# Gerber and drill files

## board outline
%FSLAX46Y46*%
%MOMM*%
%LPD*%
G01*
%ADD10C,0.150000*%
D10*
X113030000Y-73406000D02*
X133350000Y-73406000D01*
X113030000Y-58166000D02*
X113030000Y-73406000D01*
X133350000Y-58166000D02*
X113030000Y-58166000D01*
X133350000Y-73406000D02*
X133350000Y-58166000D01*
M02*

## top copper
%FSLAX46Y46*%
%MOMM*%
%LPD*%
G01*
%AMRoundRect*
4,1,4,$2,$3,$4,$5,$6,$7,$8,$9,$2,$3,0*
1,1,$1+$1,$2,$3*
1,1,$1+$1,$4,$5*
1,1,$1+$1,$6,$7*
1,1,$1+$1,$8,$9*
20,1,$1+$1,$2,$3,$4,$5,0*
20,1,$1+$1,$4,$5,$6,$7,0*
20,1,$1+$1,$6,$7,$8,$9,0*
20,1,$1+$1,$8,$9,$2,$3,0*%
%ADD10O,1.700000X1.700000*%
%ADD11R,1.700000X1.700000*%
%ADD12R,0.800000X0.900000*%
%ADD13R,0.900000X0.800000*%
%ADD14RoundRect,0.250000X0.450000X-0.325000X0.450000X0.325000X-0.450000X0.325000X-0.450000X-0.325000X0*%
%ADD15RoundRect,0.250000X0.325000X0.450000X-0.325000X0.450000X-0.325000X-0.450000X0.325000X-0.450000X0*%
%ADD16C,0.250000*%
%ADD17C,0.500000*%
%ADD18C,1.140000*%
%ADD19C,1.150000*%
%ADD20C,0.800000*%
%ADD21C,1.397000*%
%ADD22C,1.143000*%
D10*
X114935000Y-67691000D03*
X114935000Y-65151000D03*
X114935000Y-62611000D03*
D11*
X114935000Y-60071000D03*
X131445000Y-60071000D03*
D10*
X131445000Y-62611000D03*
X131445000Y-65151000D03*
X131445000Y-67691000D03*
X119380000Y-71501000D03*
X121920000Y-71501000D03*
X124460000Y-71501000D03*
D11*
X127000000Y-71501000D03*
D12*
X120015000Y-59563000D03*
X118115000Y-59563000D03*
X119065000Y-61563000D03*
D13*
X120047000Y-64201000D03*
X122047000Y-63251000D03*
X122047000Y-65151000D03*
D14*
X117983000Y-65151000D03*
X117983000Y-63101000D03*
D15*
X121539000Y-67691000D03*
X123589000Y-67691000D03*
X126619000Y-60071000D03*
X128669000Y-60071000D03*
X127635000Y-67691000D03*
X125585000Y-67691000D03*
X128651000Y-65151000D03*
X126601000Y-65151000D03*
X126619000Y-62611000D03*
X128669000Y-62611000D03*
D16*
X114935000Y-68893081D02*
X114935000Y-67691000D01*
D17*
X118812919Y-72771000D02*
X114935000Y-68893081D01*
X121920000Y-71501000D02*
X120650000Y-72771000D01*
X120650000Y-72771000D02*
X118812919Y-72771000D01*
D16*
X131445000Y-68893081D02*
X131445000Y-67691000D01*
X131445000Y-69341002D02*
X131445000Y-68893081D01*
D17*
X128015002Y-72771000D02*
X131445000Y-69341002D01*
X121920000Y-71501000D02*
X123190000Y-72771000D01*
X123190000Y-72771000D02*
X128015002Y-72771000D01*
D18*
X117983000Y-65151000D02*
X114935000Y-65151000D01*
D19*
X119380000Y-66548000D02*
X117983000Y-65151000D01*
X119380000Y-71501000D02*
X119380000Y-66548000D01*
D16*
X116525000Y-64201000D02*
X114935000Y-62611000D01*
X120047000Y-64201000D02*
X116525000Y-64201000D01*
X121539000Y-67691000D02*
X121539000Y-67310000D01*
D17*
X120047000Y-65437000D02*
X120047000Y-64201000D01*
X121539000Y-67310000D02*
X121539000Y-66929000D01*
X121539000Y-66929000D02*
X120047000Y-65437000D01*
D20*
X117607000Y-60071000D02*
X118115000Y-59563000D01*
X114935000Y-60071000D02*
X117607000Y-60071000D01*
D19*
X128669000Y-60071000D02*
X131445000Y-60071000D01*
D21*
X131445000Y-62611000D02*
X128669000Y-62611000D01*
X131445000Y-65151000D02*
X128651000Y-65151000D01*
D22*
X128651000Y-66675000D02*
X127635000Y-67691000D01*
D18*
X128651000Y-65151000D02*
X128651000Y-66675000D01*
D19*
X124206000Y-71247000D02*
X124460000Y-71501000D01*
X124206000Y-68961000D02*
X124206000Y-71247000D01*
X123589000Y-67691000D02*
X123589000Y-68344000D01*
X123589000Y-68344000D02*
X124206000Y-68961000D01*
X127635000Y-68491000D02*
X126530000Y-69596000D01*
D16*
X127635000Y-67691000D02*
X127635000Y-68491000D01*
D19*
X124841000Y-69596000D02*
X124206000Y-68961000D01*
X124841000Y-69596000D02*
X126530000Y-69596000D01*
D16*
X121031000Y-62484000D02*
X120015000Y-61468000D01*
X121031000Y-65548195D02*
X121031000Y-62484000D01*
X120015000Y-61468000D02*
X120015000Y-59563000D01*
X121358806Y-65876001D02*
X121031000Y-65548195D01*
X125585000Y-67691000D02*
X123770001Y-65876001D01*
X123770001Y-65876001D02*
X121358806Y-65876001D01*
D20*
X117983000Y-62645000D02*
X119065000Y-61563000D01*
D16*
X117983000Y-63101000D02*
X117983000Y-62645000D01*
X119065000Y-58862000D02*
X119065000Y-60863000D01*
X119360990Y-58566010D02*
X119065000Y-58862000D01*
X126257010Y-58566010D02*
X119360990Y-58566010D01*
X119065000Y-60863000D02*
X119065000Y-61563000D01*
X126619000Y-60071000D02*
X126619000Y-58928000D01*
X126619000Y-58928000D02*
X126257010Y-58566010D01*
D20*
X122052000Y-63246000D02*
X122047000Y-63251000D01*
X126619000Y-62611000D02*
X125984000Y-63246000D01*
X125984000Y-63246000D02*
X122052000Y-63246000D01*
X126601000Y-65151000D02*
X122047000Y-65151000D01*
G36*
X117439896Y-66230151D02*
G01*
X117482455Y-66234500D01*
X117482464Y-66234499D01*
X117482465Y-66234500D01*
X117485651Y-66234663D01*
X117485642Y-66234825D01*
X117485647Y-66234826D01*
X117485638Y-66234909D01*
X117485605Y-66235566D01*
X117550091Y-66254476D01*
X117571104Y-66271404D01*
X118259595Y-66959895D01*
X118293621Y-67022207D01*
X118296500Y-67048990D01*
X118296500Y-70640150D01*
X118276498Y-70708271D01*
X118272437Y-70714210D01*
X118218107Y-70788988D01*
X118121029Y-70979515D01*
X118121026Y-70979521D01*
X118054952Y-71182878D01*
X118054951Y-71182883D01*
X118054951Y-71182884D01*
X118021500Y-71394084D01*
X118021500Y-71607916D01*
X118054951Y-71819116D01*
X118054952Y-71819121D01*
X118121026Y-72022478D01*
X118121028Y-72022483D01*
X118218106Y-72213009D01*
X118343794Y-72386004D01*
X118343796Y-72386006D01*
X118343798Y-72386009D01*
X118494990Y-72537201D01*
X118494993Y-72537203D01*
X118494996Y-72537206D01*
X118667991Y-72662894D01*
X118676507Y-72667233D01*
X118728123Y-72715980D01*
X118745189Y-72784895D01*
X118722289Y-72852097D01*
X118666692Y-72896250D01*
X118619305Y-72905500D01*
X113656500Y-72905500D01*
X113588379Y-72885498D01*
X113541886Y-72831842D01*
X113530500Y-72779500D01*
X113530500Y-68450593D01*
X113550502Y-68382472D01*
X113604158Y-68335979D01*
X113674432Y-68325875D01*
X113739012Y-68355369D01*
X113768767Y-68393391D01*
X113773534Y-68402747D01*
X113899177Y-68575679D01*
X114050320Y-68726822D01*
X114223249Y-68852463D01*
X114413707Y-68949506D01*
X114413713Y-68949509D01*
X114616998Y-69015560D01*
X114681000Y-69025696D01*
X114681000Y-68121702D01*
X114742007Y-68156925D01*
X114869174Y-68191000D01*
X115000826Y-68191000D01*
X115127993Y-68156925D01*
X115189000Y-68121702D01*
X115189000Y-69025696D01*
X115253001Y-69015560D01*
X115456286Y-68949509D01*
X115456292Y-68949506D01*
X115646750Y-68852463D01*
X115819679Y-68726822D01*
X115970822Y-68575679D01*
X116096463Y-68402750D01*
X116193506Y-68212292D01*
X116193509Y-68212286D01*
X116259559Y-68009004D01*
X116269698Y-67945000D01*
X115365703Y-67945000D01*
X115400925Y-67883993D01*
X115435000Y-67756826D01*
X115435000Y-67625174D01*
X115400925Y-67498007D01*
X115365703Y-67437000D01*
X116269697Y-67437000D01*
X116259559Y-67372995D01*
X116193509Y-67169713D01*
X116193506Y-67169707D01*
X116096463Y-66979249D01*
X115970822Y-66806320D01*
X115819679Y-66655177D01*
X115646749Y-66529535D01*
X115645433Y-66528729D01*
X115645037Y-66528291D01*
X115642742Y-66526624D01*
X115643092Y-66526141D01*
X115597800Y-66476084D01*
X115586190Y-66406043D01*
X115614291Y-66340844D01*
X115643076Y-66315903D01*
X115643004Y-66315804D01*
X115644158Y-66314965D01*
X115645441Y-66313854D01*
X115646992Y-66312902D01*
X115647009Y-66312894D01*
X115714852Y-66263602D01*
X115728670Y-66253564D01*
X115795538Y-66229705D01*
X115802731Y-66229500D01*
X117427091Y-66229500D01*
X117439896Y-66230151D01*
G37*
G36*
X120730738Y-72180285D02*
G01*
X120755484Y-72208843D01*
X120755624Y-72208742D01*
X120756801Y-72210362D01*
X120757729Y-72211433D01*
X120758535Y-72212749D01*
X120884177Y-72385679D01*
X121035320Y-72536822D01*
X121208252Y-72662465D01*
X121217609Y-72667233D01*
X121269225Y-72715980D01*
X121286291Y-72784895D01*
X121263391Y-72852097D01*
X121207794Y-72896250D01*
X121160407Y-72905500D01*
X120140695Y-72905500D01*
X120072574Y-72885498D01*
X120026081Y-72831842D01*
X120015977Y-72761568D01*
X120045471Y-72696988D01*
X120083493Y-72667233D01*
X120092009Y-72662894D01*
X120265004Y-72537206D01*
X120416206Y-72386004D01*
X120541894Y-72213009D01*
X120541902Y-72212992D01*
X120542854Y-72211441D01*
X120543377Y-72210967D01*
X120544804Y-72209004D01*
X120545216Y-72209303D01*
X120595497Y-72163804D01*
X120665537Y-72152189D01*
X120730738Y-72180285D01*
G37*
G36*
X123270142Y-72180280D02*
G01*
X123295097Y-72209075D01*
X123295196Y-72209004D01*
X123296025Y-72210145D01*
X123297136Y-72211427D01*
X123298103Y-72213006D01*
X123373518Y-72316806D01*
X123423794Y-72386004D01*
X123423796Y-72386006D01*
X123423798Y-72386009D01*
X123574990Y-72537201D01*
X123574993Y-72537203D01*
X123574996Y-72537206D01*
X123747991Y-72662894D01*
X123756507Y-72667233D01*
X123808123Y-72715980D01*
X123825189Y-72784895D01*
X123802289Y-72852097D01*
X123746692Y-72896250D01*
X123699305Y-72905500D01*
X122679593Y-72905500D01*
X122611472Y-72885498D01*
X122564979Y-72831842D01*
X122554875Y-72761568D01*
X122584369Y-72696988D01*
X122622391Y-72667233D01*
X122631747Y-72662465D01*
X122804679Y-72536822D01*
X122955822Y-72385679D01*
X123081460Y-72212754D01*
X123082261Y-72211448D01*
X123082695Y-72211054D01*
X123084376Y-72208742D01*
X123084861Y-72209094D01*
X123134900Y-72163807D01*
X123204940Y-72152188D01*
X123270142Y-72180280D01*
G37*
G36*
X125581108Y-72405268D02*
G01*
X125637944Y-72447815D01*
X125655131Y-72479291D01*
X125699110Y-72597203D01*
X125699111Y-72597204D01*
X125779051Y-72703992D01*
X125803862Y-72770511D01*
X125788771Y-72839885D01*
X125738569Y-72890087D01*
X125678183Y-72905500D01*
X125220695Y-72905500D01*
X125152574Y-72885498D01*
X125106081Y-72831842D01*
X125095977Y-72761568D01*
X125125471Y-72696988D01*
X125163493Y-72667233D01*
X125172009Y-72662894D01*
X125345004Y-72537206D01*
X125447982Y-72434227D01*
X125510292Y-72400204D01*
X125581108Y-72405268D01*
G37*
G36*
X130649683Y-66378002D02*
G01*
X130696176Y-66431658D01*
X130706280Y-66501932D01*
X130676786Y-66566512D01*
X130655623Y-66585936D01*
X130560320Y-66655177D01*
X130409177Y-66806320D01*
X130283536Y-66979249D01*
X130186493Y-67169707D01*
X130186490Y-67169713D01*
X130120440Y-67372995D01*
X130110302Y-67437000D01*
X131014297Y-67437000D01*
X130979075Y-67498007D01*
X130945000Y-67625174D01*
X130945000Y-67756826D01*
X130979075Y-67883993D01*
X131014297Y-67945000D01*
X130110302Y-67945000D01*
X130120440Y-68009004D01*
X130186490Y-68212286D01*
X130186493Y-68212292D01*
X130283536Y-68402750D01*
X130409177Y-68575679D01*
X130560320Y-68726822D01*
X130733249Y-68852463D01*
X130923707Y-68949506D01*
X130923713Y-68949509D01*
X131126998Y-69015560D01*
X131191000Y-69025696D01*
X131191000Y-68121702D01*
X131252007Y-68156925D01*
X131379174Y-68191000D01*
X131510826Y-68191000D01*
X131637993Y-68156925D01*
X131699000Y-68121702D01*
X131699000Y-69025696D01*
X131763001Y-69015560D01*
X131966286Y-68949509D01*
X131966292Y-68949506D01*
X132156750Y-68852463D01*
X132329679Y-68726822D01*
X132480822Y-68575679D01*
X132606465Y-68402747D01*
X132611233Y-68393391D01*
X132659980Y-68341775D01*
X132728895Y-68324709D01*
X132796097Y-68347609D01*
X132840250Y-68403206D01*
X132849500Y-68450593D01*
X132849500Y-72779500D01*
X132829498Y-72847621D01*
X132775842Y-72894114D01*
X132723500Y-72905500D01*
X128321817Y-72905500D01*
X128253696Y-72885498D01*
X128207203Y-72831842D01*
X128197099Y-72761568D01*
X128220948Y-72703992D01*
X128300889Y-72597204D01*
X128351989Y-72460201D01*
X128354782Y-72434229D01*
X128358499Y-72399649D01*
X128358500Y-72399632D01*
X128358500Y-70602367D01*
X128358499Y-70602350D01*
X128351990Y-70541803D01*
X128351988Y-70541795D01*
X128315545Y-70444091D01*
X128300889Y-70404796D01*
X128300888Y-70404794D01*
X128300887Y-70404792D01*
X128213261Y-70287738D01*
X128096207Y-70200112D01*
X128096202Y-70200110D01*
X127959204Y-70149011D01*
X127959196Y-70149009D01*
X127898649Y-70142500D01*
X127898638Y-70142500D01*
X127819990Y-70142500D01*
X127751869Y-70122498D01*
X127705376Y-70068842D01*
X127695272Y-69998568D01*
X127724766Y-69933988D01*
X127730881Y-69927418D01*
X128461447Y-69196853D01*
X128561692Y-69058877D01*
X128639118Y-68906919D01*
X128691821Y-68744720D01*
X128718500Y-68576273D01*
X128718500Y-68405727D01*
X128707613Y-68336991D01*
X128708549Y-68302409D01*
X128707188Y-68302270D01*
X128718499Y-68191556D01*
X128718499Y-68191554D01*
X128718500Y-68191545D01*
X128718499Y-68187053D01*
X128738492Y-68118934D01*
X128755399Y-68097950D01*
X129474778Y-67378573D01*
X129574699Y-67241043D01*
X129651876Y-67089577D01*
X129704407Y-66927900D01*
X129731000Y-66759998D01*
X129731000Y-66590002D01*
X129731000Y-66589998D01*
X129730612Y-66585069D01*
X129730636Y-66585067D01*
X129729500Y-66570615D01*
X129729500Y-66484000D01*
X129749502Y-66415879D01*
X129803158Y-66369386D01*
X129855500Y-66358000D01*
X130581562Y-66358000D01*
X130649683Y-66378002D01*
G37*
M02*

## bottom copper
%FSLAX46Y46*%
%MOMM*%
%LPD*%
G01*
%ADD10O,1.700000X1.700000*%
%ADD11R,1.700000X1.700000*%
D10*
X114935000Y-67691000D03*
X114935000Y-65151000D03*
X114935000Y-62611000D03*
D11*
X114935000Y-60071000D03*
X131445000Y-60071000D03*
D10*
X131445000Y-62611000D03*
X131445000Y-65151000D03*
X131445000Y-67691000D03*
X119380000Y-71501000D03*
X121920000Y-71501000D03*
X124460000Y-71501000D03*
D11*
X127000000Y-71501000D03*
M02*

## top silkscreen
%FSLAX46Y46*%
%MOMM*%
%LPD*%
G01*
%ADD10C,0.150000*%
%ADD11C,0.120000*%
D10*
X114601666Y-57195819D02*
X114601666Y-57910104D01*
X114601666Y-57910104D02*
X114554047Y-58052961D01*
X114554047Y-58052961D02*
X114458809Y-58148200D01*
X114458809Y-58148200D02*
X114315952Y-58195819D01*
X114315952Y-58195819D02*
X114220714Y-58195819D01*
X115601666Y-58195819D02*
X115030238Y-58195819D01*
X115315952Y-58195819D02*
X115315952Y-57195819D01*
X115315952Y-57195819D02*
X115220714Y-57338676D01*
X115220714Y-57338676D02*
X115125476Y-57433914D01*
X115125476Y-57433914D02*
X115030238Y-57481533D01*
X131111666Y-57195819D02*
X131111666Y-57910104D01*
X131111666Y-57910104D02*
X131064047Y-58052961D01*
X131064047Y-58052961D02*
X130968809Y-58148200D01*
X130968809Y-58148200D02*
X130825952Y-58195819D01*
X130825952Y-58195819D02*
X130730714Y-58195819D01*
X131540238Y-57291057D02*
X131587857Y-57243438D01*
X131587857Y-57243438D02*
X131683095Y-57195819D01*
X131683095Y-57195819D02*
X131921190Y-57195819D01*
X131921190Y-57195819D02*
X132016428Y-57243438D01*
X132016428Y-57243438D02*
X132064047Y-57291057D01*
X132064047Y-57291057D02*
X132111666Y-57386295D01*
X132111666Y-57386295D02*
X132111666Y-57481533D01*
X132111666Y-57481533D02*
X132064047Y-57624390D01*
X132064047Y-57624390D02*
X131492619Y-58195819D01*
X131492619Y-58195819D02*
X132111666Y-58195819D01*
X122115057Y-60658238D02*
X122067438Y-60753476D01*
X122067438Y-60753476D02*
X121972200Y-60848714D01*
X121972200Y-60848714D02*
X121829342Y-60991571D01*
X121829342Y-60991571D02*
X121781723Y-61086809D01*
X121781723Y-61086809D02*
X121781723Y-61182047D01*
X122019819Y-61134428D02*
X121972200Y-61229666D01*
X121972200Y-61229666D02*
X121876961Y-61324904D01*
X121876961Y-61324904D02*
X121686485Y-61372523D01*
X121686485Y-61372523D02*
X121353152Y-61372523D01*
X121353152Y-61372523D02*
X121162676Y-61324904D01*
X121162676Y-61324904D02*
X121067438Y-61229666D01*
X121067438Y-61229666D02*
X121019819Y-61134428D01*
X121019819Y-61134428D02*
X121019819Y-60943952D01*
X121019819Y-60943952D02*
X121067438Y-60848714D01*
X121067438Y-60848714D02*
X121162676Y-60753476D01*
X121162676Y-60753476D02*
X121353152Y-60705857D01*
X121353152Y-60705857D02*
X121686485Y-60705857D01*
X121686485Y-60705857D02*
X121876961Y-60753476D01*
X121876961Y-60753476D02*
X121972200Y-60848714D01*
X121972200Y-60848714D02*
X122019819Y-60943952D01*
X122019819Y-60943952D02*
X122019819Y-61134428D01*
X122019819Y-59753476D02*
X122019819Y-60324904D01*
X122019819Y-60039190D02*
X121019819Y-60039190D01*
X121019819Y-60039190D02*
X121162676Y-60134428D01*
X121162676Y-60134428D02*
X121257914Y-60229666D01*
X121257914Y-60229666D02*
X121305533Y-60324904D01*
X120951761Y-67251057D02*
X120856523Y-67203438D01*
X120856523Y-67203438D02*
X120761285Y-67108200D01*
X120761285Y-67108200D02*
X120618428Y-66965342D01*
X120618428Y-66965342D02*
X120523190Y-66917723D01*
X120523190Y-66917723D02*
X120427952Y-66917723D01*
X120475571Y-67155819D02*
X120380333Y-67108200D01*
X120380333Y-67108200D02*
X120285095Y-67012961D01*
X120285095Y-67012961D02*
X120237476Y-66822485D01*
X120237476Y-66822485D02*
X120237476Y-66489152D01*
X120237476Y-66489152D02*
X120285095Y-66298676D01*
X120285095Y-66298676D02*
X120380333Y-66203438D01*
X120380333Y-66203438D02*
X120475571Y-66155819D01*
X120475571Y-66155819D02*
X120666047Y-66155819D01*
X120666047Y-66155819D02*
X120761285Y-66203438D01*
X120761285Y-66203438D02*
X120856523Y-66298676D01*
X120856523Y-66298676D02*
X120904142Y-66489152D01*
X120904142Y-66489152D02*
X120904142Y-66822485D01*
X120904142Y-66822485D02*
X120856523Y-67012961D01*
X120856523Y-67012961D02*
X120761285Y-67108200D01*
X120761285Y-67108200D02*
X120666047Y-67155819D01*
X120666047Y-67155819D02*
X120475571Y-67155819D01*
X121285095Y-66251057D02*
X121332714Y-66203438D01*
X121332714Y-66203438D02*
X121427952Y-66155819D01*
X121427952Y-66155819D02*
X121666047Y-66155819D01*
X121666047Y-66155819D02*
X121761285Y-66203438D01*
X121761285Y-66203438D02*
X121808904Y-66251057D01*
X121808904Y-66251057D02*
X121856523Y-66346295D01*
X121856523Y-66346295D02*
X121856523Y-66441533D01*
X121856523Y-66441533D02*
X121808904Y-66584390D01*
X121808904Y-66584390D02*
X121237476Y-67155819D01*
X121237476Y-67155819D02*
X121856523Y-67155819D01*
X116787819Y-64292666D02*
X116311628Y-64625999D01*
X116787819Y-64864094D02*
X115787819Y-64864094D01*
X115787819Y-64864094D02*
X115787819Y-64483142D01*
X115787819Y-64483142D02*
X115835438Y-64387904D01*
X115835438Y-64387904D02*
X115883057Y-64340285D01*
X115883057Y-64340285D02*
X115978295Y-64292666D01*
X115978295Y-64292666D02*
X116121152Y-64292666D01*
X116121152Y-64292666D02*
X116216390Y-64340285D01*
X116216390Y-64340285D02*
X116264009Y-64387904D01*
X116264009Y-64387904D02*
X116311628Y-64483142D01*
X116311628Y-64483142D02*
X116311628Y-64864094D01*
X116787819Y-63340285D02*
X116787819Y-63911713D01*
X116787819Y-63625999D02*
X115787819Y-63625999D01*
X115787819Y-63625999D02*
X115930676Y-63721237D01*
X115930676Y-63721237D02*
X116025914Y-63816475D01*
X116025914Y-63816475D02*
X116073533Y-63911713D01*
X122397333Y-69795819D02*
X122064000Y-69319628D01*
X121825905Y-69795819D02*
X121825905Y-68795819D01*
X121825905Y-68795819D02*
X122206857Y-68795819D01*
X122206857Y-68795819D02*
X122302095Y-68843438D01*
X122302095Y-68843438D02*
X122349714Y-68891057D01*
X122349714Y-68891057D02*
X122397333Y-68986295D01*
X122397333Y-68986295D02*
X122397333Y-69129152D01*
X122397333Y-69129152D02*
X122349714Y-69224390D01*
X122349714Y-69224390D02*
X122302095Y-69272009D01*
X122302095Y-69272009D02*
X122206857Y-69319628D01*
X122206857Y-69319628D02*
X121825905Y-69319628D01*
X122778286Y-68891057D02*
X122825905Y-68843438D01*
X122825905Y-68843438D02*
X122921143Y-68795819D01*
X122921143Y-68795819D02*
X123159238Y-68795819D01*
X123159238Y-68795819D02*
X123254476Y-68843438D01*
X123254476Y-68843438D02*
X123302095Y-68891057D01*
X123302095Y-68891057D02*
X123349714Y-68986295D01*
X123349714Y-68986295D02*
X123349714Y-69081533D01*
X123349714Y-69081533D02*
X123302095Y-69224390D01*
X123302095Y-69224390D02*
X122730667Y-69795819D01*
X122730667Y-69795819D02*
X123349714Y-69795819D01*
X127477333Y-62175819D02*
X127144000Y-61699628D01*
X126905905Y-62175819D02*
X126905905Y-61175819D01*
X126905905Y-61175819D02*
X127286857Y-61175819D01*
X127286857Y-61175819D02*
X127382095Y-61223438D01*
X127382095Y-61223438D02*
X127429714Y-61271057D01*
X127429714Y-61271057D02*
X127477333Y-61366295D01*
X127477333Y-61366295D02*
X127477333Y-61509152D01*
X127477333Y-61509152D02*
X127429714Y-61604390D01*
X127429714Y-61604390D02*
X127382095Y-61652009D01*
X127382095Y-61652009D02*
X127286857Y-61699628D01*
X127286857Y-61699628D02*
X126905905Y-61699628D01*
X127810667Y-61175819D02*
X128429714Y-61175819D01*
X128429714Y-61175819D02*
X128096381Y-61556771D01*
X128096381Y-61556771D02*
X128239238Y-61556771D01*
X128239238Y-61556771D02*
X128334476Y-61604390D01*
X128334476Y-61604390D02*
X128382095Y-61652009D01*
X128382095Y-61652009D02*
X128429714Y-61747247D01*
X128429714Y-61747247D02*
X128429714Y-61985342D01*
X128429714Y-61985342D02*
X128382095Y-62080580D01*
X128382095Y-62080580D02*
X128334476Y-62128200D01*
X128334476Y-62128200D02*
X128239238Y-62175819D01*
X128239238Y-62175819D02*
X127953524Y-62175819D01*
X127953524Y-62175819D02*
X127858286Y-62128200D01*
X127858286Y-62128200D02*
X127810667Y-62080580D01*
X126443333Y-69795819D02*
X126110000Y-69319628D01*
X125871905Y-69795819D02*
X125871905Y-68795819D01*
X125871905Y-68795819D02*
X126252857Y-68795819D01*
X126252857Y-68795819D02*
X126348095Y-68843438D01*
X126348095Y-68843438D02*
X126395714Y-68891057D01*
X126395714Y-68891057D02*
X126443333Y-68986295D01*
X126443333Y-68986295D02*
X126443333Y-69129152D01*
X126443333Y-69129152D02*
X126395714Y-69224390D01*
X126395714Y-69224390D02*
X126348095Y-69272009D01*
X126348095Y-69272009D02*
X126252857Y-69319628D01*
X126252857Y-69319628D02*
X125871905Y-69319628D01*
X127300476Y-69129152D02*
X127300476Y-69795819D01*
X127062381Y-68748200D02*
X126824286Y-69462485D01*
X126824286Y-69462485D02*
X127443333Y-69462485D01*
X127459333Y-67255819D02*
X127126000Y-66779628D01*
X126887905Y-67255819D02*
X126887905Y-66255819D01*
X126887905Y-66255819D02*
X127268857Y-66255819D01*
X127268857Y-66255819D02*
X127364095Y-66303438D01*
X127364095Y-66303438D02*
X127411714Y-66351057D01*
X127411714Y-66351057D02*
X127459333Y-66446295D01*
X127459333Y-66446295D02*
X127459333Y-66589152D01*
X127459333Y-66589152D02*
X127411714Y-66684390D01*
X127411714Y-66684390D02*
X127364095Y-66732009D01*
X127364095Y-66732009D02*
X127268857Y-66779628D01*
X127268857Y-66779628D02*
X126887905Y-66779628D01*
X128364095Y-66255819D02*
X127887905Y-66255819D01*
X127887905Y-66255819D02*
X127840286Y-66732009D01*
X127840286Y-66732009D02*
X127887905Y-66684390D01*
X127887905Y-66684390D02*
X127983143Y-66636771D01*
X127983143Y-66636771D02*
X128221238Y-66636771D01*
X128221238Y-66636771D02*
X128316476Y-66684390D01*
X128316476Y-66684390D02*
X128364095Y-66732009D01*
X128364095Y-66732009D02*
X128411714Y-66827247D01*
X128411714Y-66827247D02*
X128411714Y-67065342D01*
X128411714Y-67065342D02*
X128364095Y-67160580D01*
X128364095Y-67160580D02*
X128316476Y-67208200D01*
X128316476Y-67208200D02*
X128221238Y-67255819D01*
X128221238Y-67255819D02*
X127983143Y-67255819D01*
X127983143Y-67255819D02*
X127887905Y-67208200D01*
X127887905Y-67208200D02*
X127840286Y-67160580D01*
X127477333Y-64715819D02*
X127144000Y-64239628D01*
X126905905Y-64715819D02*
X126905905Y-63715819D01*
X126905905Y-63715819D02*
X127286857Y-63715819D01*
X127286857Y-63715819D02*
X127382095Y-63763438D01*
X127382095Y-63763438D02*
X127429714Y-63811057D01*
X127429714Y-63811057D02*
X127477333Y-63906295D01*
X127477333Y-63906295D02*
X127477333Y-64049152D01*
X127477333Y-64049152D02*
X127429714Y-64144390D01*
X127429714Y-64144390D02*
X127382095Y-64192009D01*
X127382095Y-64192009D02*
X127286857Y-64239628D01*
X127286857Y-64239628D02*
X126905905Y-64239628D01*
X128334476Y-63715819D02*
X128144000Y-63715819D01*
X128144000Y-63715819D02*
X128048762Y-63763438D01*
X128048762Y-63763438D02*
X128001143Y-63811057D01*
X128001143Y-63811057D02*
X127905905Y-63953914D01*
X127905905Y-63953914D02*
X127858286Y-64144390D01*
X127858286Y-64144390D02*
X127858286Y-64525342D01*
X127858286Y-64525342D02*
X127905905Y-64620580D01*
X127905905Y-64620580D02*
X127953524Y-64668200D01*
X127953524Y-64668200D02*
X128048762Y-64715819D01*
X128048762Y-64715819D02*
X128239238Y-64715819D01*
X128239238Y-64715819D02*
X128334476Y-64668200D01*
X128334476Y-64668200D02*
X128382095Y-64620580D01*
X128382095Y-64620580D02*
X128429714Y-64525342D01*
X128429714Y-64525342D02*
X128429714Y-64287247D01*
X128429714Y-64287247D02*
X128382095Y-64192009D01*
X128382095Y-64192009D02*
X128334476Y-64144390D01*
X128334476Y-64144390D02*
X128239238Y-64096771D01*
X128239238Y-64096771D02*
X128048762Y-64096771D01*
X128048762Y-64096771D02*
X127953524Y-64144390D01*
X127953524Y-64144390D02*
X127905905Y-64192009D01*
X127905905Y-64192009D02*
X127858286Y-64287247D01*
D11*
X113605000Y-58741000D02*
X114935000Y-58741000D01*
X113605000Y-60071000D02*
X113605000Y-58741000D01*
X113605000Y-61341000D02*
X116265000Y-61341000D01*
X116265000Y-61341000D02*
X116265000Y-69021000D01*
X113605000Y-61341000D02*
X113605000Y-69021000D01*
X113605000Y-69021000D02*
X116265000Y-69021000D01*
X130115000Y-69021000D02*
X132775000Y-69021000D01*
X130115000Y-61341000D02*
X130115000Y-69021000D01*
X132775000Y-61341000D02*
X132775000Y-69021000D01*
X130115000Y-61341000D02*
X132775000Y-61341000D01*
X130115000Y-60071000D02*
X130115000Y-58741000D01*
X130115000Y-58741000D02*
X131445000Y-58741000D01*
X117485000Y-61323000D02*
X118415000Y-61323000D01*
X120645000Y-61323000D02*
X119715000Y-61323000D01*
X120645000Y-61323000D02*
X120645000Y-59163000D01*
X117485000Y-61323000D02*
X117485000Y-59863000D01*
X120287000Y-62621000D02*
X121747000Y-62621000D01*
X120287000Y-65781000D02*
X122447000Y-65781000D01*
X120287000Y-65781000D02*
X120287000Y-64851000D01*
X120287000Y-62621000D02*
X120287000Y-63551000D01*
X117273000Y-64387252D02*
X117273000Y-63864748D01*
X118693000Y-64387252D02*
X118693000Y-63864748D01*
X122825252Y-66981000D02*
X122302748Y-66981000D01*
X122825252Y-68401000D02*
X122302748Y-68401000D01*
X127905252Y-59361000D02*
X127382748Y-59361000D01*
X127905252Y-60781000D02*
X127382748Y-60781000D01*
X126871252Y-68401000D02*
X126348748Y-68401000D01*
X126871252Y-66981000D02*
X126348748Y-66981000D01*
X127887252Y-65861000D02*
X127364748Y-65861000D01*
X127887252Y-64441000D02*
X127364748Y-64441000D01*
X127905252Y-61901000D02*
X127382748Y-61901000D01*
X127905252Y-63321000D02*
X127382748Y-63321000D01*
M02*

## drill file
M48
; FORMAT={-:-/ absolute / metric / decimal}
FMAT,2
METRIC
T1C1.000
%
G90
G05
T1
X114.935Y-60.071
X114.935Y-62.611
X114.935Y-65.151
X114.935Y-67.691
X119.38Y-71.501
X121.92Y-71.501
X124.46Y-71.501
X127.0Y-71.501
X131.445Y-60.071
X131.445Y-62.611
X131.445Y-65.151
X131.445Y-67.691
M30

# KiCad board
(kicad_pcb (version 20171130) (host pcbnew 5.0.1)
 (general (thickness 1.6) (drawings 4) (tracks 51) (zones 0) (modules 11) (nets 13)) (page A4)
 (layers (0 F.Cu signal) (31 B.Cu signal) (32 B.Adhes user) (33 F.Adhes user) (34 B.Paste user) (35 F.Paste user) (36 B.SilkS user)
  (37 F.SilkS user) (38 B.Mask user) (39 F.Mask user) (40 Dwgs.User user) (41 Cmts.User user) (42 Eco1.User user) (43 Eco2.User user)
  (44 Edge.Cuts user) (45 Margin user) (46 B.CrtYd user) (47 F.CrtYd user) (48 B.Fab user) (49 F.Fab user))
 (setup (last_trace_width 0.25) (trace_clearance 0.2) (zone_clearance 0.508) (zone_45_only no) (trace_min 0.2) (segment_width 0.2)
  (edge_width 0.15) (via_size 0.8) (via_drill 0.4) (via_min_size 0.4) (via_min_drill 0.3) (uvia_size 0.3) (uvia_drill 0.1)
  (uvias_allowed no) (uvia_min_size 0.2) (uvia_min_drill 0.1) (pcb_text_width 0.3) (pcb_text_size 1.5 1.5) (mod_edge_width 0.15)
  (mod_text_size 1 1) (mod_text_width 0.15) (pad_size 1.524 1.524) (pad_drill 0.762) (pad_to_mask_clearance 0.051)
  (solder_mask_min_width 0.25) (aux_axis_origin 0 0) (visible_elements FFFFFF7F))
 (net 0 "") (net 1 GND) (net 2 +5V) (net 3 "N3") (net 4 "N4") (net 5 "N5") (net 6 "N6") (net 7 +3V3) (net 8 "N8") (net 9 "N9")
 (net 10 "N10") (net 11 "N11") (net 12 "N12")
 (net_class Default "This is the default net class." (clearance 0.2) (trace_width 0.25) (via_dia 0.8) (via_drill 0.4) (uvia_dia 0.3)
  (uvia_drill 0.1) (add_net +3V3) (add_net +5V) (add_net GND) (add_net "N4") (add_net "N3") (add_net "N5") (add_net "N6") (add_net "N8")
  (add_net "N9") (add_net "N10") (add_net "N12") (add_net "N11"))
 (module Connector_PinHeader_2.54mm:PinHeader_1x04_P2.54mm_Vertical (layer F.Cu) (at 114.935 60.071)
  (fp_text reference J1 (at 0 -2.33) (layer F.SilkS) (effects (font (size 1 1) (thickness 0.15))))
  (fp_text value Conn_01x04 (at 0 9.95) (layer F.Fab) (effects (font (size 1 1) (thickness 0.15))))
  (fp_line (start -1.33 -1.33) (end 0 -1.33) (layer F.SilkS) (width 0.12))
  (fp_line (start -1.33 0) (end -1.33 -1.33) (layer F.SilkS) (width 0.12))
  (fp_line (start -1.33 1.27) (end 1.33 1.27) (layer F.SilkS) (width 0.12))
  (fp_line (start 1.33 1.27) (end 1.33 8.95) (layer F.SilkS) (width 0.12))
  (fp_line (start -1.33 1.27) (end -1.33 8.95) (layer F.SilkS) (width 0.12))
  (fp_line (start -1.33 8.95) (end 1.33 8.95) (layer F.SilkS) (width 0.12))
  (pad 4 thru_hole oval (at 0 7.62) (size 1.7 1.7) (drill 1) (layers *.Cu *.Mask) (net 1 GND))
  (pad 3 thru_hole oval (at 0 5.08) (size 1.7 1.7) (drill 1) (layers *.Cu *.Mask) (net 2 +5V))
  (pad 2 thru_hole oval (at 0 2.54) (size 1.7 1.7) (drill 1) (layers *.Cu *.Mask) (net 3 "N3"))
  (pad 1 thru_hole rect (at 0 0) (size 1.7 1.7) (drill 1) (layers *.Cu *.Mask) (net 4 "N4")))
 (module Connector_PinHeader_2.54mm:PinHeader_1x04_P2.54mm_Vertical (layer F.Cu) (at 131.445 60.071)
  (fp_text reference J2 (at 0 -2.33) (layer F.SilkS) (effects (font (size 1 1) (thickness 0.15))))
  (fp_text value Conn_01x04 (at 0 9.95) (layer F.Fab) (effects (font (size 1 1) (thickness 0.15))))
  (fp_line (start -1.33 8.95) (end 1.33 8.95) (layer F.SilkS) (width 0.12))
  (fp_line (start -1.33 1.27) (end -1.33 8.95) (layer F.SilkS) (width 0.12))
  (fp_line (start 1.33 1.27) (end 1.33 8.95) (layer F.SilkS) (width 0.12))
  (fp_line (start -1.33 1.27) (end 1.33 1.27) (layer F.SilkS) (width 0.12))
  (fp_line (start -1.33 0) (end -1.33 -1.33) (layer F.SilkS) (width 0.12))
  (fp_line (start -1.33 -1.33) (end 0 -1.33) (layer F.SilkS) (width 0.12))
  (pad 1 thru_hole rect (at 0 0) (size 1.7 1.7) (drill 1) (layers *.Cu *.Mask) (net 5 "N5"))
  (pad 2 thru_hole oval (at 0 2.54) (size 1.7 1.7) (drill 1) (layers *.Cu *.Mask) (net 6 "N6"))
  (pad 3 thru_hole oval (at 0 5.08) (size 1.7 1.7) (drill 1) (layers *.Cu *.Mask) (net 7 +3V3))
  (pad 4 thru_hole oval (at 0 7.62) (size 1.7 1.7) (drill 1) (layers *.Cu *.Mask) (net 1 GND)))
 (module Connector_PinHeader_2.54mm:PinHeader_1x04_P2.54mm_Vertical (layer B.Cu) (at 127 71.501 90)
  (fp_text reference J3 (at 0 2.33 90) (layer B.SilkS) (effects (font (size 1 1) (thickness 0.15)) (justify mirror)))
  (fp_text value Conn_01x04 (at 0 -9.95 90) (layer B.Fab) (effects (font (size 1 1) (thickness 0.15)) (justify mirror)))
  (pad 4 thru_hole oval (at 0 -7.62 90) (size 1.7 1.7) (drill 1) (layers *.Cu *.Mask) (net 2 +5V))
  (pad 3 thru_hole oval (at 0 -5.08 90) (size 1.7 1.7) (drill 1) (layers *.Cu *.Mask) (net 1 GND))
  (pad 2 thru_hole oval (at 0 -2.54 90) (size 1.7 1.7) (drill 1) (layers *.Cu *.Mask) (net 7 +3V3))
  (pad 1 thru_hole rect (at 0 0 90) (size 1.7 1.7) (drill 1) (layers *.Cu *.Mask) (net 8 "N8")))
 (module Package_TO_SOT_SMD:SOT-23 (layer F.Cu) (at 119.065 60.563 270)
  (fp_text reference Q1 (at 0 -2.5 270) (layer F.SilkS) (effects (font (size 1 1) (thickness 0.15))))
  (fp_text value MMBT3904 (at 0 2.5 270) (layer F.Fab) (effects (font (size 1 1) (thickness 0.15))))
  (fp_line (start 0.76 1.58) (end 0.76 0.65) (layer F.SilkS) (width 0.12))
  (fp_line (start 0.76 -1.58) (end 0.76 -0.65) (layer F.SilkS) (width 0.12))
  (fp_line (start 0.76 -1.58) (end -1.4 -1.58) (layer F.SilkS) (width 0.12))
  (fp_line (start 0.76 1.58) (end -0.7 1.58) (layer F.SilkS) (width 0.12))
  (pad 1 smd rect (at -1 -0.95 270) (size 0.9 0.8) (layers F.Cu F.Paste F.Mask) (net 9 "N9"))
  (pad 2 smd rect (at -1 0.95 270) (size 0.9 0.8) (layers F.Cu F.Paste F.Mask) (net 4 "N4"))
  (pad 3 smd rect (at 1 0 270) (size 0.9 0.8) (layers F.Cu F.Paste F.Mask) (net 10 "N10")))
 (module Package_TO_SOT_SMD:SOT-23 (layer F.Cu) (at 121.047 64.201 180)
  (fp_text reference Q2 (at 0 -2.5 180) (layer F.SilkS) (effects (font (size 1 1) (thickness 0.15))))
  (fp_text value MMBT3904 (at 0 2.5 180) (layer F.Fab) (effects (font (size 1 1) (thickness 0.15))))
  (fp_line (start 0.76 1.58) (end -0.7 1.58) (layer F.SilkS) (width 0.12))
  (fp_line (start 0.76 -1.58) (end -1.4 -1.58) (layer F.SilkS) (width 0.12))
  (fp_line (start 0.76 -1.58) (end 0.76 -0.65) (layer F.SilkS) (width 0.12))
  (fp_line (start 0.76 1.58) (end 0.76 0.65) (layer F.SilkS) (width 0.12))
  (pad 3 smd rect (at 1 0 180) (size 0.9 0.8) (layers F.Cu F.Paste F.Mask) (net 3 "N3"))
  (pad 2 smd rect (at -1 0.95 180) (size 0.9 0.8) (layers F.Cu F.Paste F.Mask) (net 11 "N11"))
  (pad 1 smd rect (at -1 -0.95 180) (size 0.9 0.8) (layers F.Cu F.Paste F.Mask) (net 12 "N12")))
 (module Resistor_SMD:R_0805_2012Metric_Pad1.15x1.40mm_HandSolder (layer F.Cu) (at 117.983 64.126 90)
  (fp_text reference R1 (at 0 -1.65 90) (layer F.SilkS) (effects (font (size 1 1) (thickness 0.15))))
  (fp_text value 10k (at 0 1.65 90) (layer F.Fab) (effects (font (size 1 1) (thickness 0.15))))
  (fp_line (start -0.261252 -0.71) (end 0.261252 -0.71) (layer F.SilkS) (width 0.12))
  (fp_line (start -0.261252 0.71) (end 0.261252 0.71) (layer F.SilkS) (width 0.12))
  (pad 1 smd roundrect (at -1.025 0 90) (size 1.15 1.4) (layers F.Cu F.Paste F.Mask) (roundrect_rratio 0.217391) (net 2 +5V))
  (pad 2 smd roundrect (at 1.025 0 90) (size 1.15 1.4) (layers F.Cu F.Paste F.Mask) (roundrect_rratio 0.217391) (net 10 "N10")))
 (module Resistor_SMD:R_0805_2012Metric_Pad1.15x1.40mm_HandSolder (layer F.Cu) (at 122.564 67.691 180)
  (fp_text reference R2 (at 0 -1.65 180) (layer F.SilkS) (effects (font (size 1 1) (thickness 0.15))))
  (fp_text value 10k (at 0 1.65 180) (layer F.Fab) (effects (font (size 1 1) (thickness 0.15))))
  (fp_line (start -0.261252 0.71) (end 0.261252 0.71) (layer F.SilkS) (width 0.12))
  (fp_line (start -0.261252 -0.71) (end 0.261252 -0.71) (layer F.SilkS) (width 0.12))
  (pad 2 smd roundrect (at 1.025 0 180) (size 1.15 1.4) (layers F.Cu F.Paste F.Mask) (roundrect_rratio 0.217391) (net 3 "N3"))
  (pad 1 smd roundrect (at -1.025 0 180) (size 1.15 1.4) (layers F.Cu F.Paste F.Mask) (roundrect_rratio 0.217391) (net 7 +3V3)))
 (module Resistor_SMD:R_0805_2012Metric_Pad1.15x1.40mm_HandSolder (layer F.Cu) (at 127.644 60.071 180)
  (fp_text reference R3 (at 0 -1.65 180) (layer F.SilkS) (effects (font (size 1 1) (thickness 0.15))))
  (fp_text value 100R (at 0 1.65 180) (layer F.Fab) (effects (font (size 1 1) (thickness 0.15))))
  (fp_line (start -0.261252 0.71) (end 0.261252 0.71) (layer F.SilkS) (width 0.12))
  (fp_line (start -0.261252 -0.71) (end 0.261252 -0.71) (layer F.SilkS) (width 0.12))
  (pad 2 smd roundrect (at 1.025 0 180) (size 1.15 1.4) (layers F.Cu F.Paste F.Mask) (roundrect_rratio 0.217391) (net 10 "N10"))
  (pad 1 smd roundrect (at -1.025 0 180) (size 1.15 1.4) (layers F.Cu F.Paste F.Mask) (roundrect_rratio 0.217391) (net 5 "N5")))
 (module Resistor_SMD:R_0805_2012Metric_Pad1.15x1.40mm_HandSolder (layer F.Cu) (at 126.61 67.691 180)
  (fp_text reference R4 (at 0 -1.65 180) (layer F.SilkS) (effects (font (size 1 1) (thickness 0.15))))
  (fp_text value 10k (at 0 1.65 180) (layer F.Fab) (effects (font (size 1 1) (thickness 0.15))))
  (fp_line (start -0.261252 -0.71) (end 0.261252 -0.71) (layer F.SilkS) (width 0.12))
  (fp_line (start -0.261252 0.71) (end 0.261252 0.71) (layer F.SilkS) (width 0.12))
  (pad 1 smd roundrect (at -1.025 0 180) (size 1.15 1.4) (layers F.Cu F.Paste F.Mask) (roundrect_rratio 0.217391) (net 7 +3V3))
  (pad 2 smd roundrect (at 1.025 0 180) (size 1.15 1.4) (layers F.Cu F.Paste F.Mask) (roundrect_rratio 0.217391) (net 9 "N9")))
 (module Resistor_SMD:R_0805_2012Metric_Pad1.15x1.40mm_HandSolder (layer F.Cu) (at 127.626 65.151 180)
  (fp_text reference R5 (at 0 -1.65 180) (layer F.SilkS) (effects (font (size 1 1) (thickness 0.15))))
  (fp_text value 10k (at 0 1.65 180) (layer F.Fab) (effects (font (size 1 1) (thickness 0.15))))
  (fp_line (start -0.261252 -0.71) (end 0.261252 -0.71) (layer F.SilkS) (width 0.12))
  (fp_line (start -0.261252 0.71) (end 0.261252 0.71) (layer F.SilkS) (width 0.12))
  (pad 1 smd roundrect (at -1.025 0 180) (size 1.15 1.4) (layers F.Cu F.Paste F.Mask) (roundrect_rratio 0.217391) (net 7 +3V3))
  (pad 2 smd roundrect (at 1.025 0 180) (size 1.15 1.4) (layers F.Cu F.Paste F.Mask) (roundrect_rratio 0.217391) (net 12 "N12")))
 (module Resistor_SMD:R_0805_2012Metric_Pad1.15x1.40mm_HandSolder (layer F.Cu) (at 127.644 62.611 180)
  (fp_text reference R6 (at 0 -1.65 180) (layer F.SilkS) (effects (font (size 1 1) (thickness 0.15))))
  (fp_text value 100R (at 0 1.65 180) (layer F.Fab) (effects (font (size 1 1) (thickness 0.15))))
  (fp_line (start -0.261252 0.71) (end 0.261252 0.71) (layer F.SilkS) (width 0.12))
  (fp_line (start -0.261252 -0.71) (end 0.261252 -0.71) (layer F.SilkS) (width 0.12))
  (pad 2 smd roundrect (at 1.025 0 180) (size 1.15 1.4) (layers F.Cu F.Paste F.Mask) (roundrect_rratio 0.217391) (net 11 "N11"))
  (pad 1 smd roundrect (at -1.025 0 180) (size 1.15 1.4) (layers F.Cu F.Paste F.Mask) (roundrect_rratio 0.217391) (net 6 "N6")))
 (gr_line (start 113.03 73.406) (end 133.35 73.406) (layer Edge.Cuts) (width 0.15))
 (gr_line (start 113.03 58.166) (end 113.03 73.406) (layer Edge.Cuts) (width 0.15))
 (gr_line (start 133.35 58.166) (end 113.03 58.166) (layer Edge.Cuts) (width 0.15))
 (gr_line (start 133.35 73.406) (end 133.35 58.166) (layer Edge.Cuts) (width 0.15))
 (segment (start 114.935 68.893081) (end 114.935 67.691) (width 0.25) (layer F.Cu) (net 1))
 (segment (start 118.812919 72.771) (end 114.935 68.893081) (width 0.5) (layer F.Cu) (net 1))
 (segment (start 121.92 71.501) (end 120.65 72.771) (width 0.5) (layer F.Cu) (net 1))
 (segment (start 120.65 72.771) (end 118.812919 72.771) (width 0.5) (layer F.Cu) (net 1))
 (segment (start 131.445 68.893081) (end 131.445 67.691) (width 0.25) (layer F.Cu) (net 1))
 (segment (start 131.445 69.341002) (end 131.445 68.893081) (width 0.25) (layer F.Cu) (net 1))
 (segment (start 128.015002 72.771) (end 131.445 69.341002) (width 0.5) (layer F.Cu) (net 1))
 (segment (start 121.92 71.501) (end 123.19 72.771) (width 0.5) (layer F.Cu) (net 1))
 (segment (start 123.19 72.771) (end 128.015002 72.771) (width 0.5) (layer F.Cu) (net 1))
 (segment (start 117.983 65.151) (end 114.935 65.151) (width 1.14) (layer F.Cu) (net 2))
 (segment (start 119.38 66.548) (end 117.983 65.151) (width 1.15) (layer F.Cu) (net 2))
 (segment (start 119.38 71.501) (end 119.38 66.548) (width 1.15) (layer F.Cu) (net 2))
 (segment (start 116.525 64.201) (end 114.935 62.611) (width 0.25) (layer F.Cu) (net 3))
 (segment (start 120.047 64.201) (end 116.525 64.201) (width 0.25) (layer F.Cu) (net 3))
 (segment (start 121.539 67.691) (end 121.539 67.31) (width 0.25) (layer F.Cu) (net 3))
 (segment (start 120.047 65.437) (end 120.047 64.201) (width 0.5) (layer F.Cu) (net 3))
 (segment (start 121.539 67.31) (end 121.539 66.929) (width 0.5) (layer F.Cu) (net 3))
 (segment (start 121.539 66.929) (end 120.047 65.437) (width 0.5) (layer F.Cu) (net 3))
 (segment (start 117.607 60.071) (end 118.115 59.563) (width 0.8) (layer F.Cu) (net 4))
 (segment (start 114.935 60.071) (end 117.607 60.071) (width 0.8) (layer F.Cu) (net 4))
 (segment (start 128.669 60.071) (end 131.445 60.071) (width 1.15) (layer F.Cu) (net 5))
 (segment (start 131.445 62.611) (end 128.669 62.611) (width 1.397) (layer F.Cu) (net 6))
 (segment (start 131.445 65.151) (end 128.651 65.151) (width 1.397) (layer F.Cu) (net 7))
 (segment (start 128.651 66.675) (end 127.635 67.691) (width 1.143) (layer F.Cu) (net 7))
 (segment (start 128.651 65.151) (end 128.651 66.675) (width 1.14) (layer F.Cu) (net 7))
 (segment (start 124.206 71.247) (end 124.46 71.501) (width 1.15) (layer F.Cu) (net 7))
 (segment (start 124.206 68.961) (end 124.206 71.247) (width 1.15) (layer F.Cu) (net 7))
 (segment (start 123.589 67.691) (end 123.589 68.344) (width 1.15) (layer F.Cu) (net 7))
 (segment (start 123.589 68.344) (end 124.206 68.961) (width 1.15) (layer F.Cu) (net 7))
 (segment (start 127.635 68.491) (end 126.53 69.596) (width 1.15) (layer F.Cu) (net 7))
 (segment (start 127.635 67.691) (end 127.635 68.491) (width 0.25) (layer F.Cu) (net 7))
 (segment (start 124.841 69.596) (end 124.206 68.961) (width 1.15) (layer F.Cu) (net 7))
 (segment (start 124.841 69.596) (end 126.53 69.596) (width 1.15) (layer F.Cu) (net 7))
 (segment (start 121.031 62.484) (end 120.015 61.468) (width 0.25) (layer F.Cu) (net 9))
 (segment (start 121.031 65.548195) (end 121.031 62.484) (width 0.25) (layer F.Cu) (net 9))
 (segment (start 120.015 61.468) (end 120.015 59.563) (width 0.25) (layer F.Cu) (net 9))
 (segment (start 121.358806 65.876001) (end 121.031 65.548195) (width 0.25) (layer F.Cu) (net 9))
 (segment (start 125.585 67.691) (end 123.770001 65.876001) (width 0.25) (layer F.Cu) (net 9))
 (segment (start 123.770001 65.876001) (end 121.358806 65.876001) (width 0.25) (layer F.Cu) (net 9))
 (segment (start 117.983 62.645) (end 119.065 61.563) (width 0.8) (layer F.Cu) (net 10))
 (segment (start 117.983 63.101) (end 117.983 62.645) (width 0.25) (layer F.Cu) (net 10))
 (segment (start 119.065 58.862) (end 119.065 60.863) (width 0.25) (layer F.Cu) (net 10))
 (segment (start 119.36099 58.56601) (end 119.065 58.862) (width 0.25) (layer F.Cu) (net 10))
 (segment (start 126.25701 58.56601) (end 119.36099 58.56601) (width 0.25) (layer F.Cu) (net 10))
 (segment (start 119.065 60.863) (end 119.065 61.563) (width 0.25) (layer F.Cu) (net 10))
 (segment (start 126.619 60.071) (end 126.619 58.928) (width 0.25) (layer F.Cu) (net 10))
 (segment (start 126.619 58.928) (end 126.25701 58.56601) (width 0.25) (layer F.Cu) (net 10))
 (segment (start 122.052 63.246) (end 122.047 63.251) (width 0.8) (layer F.Cu) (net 11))
 (segment (start 126.619 62.611) (end 125.984 63.246) (width 0.8) (layer F.Cu) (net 11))
 (segment (start 125.984 63.246) (end 122.052 63.246) (width 0.8) (layer F.Cu) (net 11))
 (segment (start 126.601 65.151) (end 122.047 65.151) (width 0.8) (layer F.Cu) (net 12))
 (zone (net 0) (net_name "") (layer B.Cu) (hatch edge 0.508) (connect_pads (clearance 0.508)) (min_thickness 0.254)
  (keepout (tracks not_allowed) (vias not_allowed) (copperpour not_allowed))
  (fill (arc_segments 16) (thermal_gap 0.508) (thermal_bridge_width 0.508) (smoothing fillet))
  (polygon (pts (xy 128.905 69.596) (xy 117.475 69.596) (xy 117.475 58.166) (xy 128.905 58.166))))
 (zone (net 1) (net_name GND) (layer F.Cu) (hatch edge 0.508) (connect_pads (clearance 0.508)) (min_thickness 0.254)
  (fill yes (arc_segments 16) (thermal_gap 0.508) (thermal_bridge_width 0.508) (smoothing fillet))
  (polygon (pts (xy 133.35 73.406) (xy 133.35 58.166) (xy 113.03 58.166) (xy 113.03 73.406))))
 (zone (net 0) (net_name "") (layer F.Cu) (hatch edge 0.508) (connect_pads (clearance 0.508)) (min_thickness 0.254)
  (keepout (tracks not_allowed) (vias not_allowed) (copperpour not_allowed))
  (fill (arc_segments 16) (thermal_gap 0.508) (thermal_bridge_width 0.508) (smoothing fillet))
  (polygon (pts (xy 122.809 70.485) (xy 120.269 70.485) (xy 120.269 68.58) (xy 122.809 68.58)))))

